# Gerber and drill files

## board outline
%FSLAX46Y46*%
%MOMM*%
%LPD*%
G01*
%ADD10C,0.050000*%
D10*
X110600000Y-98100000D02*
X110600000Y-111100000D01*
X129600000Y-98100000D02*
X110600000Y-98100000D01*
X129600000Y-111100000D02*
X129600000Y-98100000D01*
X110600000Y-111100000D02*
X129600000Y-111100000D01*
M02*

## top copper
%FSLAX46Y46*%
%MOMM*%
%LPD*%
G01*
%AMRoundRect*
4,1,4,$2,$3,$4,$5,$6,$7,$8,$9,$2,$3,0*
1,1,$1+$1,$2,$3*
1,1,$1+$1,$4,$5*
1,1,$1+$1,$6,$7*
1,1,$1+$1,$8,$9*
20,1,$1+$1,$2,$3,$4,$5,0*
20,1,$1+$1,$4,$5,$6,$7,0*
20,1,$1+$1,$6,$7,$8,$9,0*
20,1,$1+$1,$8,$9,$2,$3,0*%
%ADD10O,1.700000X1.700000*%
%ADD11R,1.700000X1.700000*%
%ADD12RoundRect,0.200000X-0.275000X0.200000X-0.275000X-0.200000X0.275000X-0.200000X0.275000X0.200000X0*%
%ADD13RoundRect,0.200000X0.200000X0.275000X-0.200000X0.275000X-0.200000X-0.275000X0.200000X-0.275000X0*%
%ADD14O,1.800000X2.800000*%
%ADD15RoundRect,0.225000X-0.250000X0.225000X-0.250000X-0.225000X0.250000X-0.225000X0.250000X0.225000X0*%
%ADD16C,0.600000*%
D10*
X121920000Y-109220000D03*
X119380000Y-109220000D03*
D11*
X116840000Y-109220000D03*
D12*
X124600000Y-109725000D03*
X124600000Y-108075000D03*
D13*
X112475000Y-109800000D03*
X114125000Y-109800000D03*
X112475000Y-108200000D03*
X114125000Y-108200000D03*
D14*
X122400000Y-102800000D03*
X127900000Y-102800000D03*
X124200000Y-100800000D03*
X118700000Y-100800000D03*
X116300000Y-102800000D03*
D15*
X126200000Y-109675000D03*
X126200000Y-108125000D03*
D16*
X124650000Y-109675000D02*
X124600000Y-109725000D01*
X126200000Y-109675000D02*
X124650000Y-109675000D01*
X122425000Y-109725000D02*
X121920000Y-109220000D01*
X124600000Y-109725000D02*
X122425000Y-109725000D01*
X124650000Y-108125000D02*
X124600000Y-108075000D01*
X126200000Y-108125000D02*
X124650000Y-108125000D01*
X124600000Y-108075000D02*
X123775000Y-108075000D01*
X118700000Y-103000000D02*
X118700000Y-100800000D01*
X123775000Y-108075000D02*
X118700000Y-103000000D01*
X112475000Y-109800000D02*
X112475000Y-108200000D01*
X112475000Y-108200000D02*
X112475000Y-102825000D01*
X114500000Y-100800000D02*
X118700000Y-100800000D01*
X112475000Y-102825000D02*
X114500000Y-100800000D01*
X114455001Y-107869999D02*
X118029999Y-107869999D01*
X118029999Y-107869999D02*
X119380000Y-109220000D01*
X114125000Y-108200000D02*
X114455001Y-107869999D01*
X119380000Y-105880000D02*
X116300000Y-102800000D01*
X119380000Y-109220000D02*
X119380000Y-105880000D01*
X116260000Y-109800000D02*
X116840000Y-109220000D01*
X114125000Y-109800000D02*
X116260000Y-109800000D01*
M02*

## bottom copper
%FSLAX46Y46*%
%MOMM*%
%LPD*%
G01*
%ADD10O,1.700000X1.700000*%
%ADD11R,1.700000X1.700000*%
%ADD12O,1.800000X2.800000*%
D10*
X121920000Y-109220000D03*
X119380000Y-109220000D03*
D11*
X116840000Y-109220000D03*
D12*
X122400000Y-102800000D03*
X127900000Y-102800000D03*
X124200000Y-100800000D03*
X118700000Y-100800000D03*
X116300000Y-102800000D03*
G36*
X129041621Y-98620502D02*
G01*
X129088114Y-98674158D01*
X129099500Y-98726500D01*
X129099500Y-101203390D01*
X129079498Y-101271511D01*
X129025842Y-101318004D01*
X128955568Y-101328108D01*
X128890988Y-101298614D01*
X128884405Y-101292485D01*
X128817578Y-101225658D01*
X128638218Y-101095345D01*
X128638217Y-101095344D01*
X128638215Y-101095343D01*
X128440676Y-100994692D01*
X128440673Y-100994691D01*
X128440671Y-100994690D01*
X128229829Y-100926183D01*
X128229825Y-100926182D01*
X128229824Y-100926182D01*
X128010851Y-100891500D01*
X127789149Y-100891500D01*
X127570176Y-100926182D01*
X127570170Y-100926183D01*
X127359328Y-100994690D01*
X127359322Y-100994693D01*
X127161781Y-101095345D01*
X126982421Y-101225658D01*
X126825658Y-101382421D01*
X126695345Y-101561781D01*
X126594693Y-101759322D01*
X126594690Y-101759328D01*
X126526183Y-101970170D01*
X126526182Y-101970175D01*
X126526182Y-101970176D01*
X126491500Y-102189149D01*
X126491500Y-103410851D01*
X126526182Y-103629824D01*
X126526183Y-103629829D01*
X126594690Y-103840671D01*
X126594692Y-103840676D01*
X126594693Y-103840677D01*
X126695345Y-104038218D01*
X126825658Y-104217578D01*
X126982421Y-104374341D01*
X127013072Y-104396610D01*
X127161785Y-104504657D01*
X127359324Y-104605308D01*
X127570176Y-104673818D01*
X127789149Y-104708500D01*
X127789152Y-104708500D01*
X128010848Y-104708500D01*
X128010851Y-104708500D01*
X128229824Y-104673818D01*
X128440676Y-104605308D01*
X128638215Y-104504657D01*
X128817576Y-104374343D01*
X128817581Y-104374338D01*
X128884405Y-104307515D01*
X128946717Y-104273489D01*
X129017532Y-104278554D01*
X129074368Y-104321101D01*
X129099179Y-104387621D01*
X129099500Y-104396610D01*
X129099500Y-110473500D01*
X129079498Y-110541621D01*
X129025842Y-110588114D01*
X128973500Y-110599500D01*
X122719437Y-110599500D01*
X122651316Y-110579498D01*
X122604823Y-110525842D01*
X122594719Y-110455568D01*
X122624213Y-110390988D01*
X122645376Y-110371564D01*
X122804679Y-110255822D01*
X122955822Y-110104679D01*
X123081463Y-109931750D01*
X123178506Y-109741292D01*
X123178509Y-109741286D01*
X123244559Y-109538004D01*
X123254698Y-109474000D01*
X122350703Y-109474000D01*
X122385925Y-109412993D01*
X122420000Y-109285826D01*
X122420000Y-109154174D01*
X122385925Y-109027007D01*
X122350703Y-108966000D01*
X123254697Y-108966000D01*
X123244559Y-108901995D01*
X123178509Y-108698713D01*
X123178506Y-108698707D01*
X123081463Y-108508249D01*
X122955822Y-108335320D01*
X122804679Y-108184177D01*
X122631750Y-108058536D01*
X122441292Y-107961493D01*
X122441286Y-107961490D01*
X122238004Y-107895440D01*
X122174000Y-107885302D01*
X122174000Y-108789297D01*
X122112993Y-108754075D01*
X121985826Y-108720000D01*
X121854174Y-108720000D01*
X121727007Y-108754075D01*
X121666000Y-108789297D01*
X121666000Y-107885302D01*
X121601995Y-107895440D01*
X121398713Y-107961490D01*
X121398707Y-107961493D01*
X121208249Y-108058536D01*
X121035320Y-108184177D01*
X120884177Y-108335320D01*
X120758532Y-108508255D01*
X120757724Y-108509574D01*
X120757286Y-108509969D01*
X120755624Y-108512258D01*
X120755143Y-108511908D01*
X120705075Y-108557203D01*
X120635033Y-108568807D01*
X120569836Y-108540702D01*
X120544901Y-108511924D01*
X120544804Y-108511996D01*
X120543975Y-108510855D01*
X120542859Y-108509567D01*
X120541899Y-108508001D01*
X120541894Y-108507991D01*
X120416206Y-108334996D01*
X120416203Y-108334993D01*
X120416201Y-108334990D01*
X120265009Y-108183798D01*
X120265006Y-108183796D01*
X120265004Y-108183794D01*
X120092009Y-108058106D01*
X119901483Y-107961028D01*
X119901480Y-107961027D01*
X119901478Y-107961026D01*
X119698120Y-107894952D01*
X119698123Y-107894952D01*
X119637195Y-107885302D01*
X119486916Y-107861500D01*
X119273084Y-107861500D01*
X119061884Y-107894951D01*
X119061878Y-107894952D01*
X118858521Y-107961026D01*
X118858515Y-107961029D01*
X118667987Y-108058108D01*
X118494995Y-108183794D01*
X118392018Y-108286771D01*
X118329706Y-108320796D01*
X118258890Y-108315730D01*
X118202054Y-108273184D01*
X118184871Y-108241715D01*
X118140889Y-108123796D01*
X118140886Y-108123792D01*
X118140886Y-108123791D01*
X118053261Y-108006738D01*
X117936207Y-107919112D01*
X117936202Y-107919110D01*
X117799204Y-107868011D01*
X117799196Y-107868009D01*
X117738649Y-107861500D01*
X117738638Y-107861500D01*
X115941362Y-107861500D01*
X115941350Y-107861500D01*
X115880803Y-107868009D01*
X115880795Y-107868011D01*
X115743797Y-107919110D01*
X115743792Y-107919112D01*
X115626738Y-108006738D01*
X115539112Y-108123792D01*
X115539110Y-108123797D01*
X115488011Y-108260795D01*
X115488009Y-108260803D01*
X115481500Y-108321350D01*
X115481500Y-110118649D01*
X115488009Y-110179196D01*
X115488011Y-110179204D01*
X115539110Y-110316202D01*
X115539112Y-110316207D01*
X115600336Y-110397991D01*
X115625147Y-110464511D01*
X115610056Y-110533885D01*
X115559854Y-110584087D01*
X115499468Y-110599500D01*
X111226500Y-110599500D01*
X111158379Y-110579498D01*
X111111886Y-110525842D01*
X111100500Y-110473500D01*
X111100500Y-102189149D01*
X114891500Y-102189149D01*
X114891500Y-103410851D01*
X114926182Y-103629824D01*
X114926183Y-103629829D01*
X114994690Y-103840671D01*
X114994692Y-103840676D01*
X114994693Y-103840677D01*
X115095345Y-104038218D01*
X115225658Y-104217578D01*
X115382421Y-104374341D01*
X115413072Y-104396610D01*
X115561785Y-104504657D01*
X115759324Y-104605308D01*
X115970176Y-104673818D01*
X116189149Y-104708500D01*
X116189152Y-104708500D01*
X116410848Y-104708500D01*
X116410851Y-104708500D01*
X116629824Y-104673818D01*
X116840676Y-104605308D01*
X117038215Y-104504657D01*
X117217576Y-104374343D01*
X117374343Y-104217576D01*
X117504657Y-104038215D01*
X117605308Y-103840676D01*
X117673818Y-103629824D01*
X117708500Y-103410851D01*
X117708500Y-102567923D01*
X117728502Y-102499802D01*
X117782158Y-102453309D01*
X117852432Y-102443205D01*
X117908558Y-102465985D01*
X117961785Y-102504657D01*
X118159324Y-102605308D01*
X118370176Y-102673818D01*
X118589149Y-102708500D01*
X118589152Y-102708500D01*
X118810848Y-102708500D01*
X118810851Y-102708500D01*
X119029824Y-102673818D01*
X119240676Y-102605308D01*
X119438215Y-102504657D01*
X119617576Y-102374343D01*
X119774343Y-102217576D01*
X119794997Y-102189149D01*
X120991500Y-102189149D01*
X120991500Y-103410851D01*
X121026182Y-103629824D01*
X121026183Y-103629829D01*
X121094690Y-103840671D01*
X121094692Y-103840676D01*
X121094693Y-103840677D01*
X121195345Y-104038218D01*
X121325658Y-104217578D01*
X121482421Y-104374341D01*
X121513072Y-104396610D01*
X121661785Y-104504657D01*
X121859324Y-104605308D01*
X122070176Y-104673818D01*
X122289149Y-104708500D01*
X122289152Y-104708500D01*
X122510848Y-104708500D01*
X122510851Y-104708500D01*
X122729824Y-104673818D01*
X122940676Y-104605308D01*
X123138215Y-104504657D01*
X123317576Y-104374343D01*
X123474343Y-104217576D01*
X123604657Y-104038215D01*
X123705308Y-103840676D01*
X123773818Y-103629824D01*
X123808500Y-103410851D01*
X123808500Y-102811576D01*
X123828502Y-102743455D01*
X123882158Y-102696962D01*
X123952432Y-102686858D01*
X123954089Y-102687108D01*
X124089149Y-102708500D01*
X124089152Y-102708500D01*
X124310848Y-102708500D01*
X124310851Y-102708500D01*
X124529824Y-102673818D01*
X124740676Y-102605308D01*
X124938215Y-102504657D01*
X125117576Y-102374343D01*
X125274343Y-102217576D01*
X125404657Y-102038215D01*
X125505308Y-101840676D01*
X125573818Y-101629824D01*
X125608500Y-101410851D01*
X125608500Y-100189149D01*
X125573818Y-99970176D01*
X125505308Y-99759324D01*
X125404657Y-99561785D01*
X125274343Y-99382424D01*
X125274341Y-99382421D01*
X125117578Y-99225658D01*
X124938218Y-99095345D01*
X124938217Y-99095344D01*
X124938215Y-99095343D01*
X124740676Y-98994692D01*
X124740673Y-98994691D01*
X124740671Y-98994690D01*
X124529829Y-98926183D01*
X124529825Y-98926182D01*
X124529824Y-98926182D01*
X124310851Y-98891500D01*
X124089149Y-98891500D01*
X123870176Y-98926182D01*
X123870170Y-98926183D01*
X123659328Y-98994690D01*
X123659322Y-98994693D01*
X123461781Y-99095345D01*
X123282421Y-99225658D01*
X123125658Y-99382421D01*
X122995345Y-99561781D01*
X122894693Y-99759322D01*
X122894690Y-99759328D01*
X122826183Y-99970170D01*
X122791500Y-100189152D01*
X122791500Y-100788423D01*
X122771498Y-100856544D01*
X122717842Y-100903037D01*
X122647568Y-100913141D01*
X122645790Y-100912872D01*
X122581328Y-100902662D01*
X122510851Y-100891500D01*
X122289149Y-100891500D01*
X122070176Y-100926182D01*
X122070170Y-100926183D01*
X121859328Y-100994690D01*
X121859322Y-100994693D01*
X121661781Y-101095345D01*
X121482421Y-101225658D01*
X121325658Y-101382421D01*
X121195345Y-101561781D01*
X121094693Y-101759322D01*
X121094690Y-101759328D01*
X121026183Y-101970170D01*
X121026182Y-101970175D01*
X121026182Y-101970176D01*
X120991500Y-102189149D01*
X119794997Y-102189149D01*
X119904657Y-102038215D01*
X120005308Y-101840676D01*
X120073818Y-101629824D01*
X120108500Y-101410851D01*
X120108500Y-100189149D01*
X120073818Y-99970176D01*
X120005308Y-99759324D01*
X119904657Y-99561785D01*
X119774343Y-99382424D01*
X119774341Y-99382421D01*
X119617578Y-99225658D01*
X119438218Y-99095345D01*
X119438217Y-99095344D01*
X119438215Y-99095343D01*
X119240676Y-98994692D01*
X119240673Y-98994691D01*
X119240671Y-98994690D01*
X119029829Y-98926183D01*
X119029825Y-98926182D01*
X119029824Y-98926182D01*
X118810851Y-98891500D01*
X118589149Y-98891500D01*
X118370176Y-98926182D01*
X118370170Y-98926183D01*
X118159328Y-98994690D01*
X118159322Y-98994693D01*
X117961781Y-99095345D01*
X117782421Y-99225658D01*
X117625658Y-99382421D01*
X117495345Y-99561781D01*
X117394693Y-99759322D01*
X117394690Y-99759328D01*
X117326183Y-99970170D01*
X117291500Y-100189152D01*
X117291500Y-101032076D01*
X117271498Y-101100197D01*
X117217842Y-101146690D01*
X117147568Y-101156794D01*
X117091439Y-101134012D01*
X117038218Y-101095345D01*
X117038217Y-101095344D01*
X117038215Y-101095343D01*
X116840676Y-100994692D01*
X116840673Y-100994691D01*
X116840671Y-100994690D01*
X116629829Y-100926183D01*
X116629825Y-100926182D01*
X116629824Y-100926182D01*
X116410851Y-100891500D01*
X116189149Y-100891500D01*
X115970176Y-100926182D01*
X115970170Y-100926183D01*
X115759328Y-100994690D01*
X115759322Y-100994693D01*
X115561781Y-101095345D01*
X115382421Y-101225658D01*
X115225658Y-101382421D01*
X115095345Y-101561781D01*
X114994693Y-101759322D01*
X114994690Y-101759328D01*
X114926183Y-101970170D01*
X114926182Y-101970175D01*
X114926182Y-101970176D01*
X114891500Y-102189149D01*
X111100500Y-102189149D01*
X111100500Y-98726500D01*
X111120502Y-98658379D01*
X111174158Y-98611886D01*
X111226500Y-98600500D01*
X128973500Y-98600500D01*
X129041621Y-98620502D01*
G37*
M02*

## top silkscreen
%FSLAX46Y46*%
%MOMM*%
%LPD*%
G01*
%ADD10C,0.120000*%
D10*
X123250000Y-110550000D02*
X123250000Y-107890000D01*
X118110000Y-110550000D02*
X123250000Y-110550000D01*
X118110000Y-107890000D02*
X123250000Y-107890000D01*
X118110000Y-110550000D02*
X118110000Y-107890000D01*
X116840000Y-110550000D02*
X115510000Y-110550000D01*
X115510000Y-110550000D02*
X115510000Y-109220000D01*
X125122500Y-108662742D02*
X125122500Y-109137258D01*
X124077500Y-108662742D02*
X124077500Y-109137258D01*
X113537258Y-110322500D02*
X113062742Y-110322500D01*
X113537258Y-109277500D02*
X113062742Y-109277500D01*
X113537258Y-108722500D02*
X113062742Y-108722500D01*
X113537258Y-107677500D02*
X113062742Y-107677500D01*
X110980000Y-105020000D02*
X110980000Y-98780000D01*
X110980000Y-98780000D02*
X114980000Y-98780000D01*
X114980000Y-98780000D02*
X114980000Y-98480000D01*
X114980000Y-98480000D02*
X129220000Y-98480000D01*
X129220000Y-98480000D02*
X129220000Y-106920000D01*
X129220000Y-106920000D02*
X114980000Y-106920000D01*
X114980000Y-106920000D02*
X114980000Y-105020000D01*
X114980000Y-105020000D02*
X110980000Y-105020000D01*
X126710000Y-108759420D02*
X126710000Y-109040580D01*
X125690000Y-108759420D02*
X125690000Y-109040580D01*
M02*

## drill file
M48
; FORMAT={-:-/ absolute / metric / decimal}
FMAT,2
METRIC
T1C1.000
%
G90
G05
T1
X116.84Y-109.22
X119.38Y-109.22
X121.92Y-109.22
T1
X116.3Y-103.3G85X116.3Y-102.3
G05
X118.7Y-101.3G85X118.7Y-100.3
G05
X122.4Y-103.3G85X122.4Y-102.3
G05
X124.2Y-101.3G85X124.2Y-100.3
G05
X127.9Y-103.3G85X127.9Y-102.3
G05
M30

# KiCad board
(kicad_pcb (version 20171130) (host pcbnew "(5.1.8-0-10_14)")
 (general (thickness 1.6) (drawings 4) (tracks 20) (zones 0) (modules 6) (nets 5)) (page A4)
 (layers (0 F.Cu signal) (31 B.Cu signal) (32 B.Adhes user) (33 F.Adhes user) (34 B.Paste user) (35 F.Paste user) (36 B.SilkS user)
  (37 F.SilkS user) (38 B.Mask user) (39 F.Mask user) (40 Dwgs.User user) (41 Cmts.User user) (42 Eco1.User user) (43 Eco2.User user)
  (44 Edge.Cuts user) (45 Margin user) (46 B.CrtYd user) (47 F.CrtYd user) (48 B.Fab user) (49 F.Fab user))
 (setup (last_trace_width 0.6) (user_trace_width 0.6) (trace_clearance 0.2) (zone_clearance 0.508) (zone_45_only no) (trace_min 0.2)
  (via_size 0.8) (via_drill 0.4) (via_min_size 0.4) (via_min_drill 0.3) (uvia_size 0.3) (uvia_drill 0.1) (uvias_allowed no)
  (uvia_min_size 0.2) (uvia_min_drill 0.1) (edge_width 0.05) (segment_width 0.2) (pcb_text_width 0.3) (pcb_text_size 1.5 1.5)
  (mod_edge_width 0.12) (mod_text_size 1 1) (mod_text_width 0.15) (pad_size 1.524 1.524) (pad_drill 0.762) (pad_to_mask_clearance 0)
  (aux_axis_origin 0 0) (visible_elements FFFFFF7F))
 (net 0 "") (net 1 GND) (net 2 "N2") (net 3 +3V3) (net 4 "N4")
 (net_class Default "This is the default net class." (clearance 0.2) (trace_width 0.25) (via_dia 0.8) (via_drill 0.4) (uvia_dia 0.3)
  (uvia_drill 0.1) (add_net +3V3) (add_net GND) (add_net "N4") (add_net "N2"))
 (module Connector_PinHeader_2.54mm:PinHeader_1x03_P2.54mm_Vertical (layer F.Cu) (at 116.84 109.22 90)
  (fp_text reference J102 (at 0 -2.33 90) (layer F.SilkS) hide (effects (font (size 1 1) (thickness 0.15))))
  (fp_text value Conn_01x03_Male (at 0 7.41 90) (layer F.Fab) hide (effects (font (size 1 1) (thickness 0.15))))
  (fp_line (start -1.33 6.41) (end 1.33 6.41) (layer F.SilkS) (width 0.12))
  (fp_line (start -1.33 1.27) (end -1.33 6.41) (layer F.SilkS) (width 0.12))
  (fp_line (start 1.33 1.27) (end 1.33 6.41) (layer F.SilkS) (width 0.12))
  (fp_line (start -1.33 1.27) (end 1.33 1.27) (layer F.SilkS) (width 0.12))
  (fp_line (start -1.33 0) (end -1.33 -1.33) (layer F.SilkS) (width 0.12))
  (fp_line (start -1.33 -1.33) (end 0 -1.33) (layer F.SilkS) (width 0.12))
  (pad 3 thru_hole oval (at 0 5.08 90) (size 1.7 1.7) (drill 1) (layers *.Cu *.Mask) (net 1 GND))
  (pad 2 thru_hole oval (at 0 2.54 90) (size 1.7 1.7) (drill 1) (layers *.Cu *.Mask) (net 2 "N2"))
  (pad 1 thru_hole rect (at 0 0 90) (size 1.7 1.7) (drill 1) (layers *.Cu *.Mask) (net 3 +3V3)))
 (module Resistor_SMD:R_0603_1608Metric (layer F.Cu) (at 124.6 108.9 270)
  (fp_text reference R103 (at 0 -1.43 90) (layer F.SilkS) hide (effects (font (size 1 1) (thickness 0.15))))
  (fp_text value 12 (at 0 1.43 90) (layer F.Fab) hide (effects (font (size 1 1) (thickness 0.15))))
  (fp_line (start -0.237258 -0.5225) (end 0.237258 -0.5225) (layer F.SilkS) (width 0.12))
  (fp_line (start -0.237258 0.5225) (end 0.237258 0.5225) (layer F.SilkS) (width 0.12))
  (pad 2 smd roundrect (at 0.825 0 270) (size 0.8 0.95) (layers F.Cu F.Paste F.Mask) (roundrect_rratio 0.25) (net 1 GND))
  (pad 1 smd roundrect (at -0.825 0 270) (size 0.8 0.95) (layers F.Cu F.Paste F.Mask) (roundrect_rratio 0.25) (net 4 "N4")))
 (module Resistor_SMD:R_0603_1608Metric (layer F.Cu) (at 113.3 109.8 180)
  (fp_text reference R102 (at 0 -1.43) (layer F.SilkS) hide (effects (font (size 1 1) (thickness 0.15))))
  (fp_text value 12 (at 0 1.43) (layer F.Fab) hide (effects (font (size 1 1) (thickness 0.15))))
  (fp_line (start -0.237258 -0.5225) (end 0.237258 -0.5225) (layer F.SilkS) (width 0.12))
  (fp_line (start -0.237258 0.5225) (end 0.237258 0.5225) (layer F.SilkS) (width 0.12))
  (pad 2 smd roundrect (at 0.825 0 180) (size 0.8 0.95) (layers F.Cu F.Paste F.Mask) (roundrect_rratio 0.25) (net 4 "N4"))
  (pad 1 smd roundrect (at -0.825 0 180) (size 0.8 0.95) (layers F.Cu F.Paste F.Mask) (roundrect_rratio 0.25) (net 3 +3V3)))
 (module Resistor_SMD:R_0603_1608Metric (layer F.Cu) (at 113.3 108.2 180)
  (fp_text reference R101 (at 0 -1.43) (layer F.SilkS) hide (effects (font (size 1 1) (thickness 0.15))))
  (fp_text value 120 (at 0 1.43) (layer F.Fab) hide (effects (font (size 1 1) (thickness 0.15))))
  (fp_line (start -0.237258 -0.5225) (end 0.237258 -0.5225) (layer F.SilkS) (width 0.12))
  (fp_line (start -0.237258 0.5225) (end 0.237258 0.5225) (layer F.SilkS) (width 0.12))
  (pad 2 smd roundrect (at 0.825 0 180) (size 0.8 0.95) (layers F.Cu F.Paste F.Mask) (roundrect_rratio 0.25) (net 4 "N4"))
  (pad 1 smd roundrect (at -0.825 0 180) (size 0.8 0.95) (layers F.Cu F.Paste F.Mask) (roundrect_rratio 0.25) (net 2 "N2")))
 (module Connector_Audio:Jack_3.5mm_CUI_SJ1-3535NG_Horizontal (layer F.Cu) (at 116.3 102.8 90)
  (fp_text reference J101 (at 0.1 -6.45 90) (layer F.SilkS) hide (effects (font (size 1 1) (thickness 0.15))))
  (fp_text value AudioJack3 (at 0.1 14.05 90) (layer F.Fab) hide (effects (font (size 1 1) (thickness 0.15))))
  (fp_line (start -2.22 -5.32) (end 4.02 -5.32) (layer F.SilkS) (width 0.12))
  (fp_line (start 4.02 -5.32) (end 4.02 -1.32) (layer F.SilkS) (width 0.12))
  (fp_line (start 4.02 -1.32) (end 4.32 -1.32) (layer F.SilkS) (width 0.12))
  (fp_line (start 4.32 -1.32) (end 4.32 12.92) (layer F.SilkS) (width 0.12))
  (fp_line (start 4.32 12.92) (end -4.12 12.92) (layer F.SilkS) (width 0.12))
  (fp_line (start -4.12 12.92) (end -4.12 -1.32) (layer F.SilkS) (width 0.12))
  (fp_line (start -4.12 -1.32) (end -2.22 -1.32) (layer F.SilkS) (width 0.12))
  (fp_line (start -2.22 -1.32) (end -2.22 -5.32) (layer F.SilkS) (width 0.12))
  (pad RN thru_hole oval (at 0 6.1 90) (size 2.8 1.8) (drill oval 2 1) (layers *.Cu *.Mask))
  (pad TN thru_hole oval (at 0 11.6 90) (size 2.8 1.8) (drill oval 2 1) (layers *.Cu *.Mask))
  (pad R thru_hole oval (at 2 7.9 90) (size 2.8 1.8) (drill oval 2 1) (layers *.Cu *.Mask))
  (pad T thru_hole oval (at 2 2.4 90) (size 2.8 1.8) (drill oval 2 1) (layers *.Cu *.Mask) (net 4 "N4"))
  (pad S thru_hole oval (at 0 0 90) (size 2.8 1.8) (drill oval 2 1) (layers *.Cu *.Mask) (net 2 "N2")))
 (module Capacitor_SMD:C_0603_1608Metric (layer F.Cu) (at 126.2 108.9 270)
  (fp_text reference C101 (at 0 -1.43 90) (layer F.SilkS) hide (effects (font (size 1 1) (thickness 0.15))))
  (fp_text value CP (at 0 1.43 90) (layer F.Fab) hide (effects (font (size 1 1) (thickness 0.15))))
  (fp_line (start -0.14058 -0.51) (end 0.14058 -0.51) (layer F.SilkS) (width 0.12))
  (fp_line (start -0.14058 0.51) (end 0.14058 0.51) (layer F.SilkS) (width 0.12))
  (pad 2 smd roundrect (at 0.775 0 270) (size 0.9 0.95) (layers F.Cu F.Paste F.Mask) (roundrect_rratio 0.25) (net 1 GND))
  (pad 1 smd roundrect (at -0.775 0 270) (size 0.9 0.95) (layers F.Cu F.Paste F.Mask) (roundrect_rratio 0.25) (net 4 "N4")))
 (gr_line (start 110.6 98.1) (end 110.6 111.1) (layer Edge.Cuts) (width 0.05))
 (gr_line (start 129.6 98.1) (end 110.6 98.1) (layer Edge.Cuts) (width 0.05))
 (gr_line (start 129.6 111.1) (end 129.6 98.1) (layer Edge.Cuts) (width 0.05))
 (gr_line (start 110.6 111.1) (end 129.6 111.1) (layer Edge.Cuts) (width 0.05))
 (segment (start 124.65 109.675) (end 124.6 109.725) (width 0.6) (layer F.Cu) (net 1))
 (segment (start 126.2 109.675) (end 124.65 109.675) (width 0.6) (layer F.Cu) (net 1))
 (segment (start 122.425 109.725) (end 121.92 109.22) (width 0.6) (layer F.Cu) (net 1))
 (segment (start 124.6 109.725) (end 122.425 109.725) (width 0.6) (layer F.Cu) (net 1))
 (segment (start 124.65 108.125) (end 124.6 108.075) (width 0.6) (layer F.Cu) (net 4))
 (segment (start 126.2 108.125) (end 124.65 108.125) (width 0.6) (layer F.Cu) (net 4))
 (segment (start 124.6 108.075) (end 123.775 108.075) (width 0.6) (layer F.Cu) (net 4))
 (segment (start 118.7 103) (end 118.7 100.8) (width 0.6) (layer F.Cu) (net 4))
 (segment (start 123.775 108.075) (end 118.7 103) (width 0.6) (layer F.Cu) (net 4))
 (segment (start 112.475 109.8) (end 112.475 108.2) (width 0.6) (layer F.Cu) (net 4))
 (segment (start 112.475 108.2) (end 112.475 102.825) (width 0.6) (layer F.Cu) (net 4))
 (segment (start 114.5 100.8) (end 118.7 100.8) (width 0.6) (layer F.Cu) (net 4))
 (segment (start 112.475 102.825) (end 114.5 100.8) (width 0.6) (layer F.Cu) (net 4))
 (segment (start 114.455001 107.869999) (end 118.029999 107.869999) (width 0.6) (layer F.Cu) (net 2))
 (segment (start 118.029999 107.869999) (end 119.38 109.22) (width 0.6) (layer F.Cu) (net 2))
 (segment (start 114.125 108.2) (end 114.455001 107.869999) (width 0.6) (layer F.Cu) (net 2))
 (segment (start 119.38 105.88) (end 116.3 102.8) (width 0.6) (layer F.Cu) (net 2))
 (segment (start 119.38 109.22) (end 119.38 105.88) (width 0.6) (layer F.Cu) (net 2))
 (segment (start 116.26 109.8) (end 116.84 109.22) (width 0.6) (layer F.Cu) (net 3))
 (segment (start 114.125 109.8) (end 116.26 109.8) (width 0.6) (layer F.Cu) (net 3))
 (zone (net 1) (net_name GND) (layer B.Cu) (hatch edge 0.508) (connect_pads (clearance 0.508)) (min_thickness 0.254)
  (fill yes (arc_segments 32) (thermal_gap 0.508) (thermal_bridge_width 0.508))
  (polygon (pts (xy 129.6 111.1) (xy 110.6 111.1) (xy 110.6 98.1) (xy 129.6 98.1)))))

